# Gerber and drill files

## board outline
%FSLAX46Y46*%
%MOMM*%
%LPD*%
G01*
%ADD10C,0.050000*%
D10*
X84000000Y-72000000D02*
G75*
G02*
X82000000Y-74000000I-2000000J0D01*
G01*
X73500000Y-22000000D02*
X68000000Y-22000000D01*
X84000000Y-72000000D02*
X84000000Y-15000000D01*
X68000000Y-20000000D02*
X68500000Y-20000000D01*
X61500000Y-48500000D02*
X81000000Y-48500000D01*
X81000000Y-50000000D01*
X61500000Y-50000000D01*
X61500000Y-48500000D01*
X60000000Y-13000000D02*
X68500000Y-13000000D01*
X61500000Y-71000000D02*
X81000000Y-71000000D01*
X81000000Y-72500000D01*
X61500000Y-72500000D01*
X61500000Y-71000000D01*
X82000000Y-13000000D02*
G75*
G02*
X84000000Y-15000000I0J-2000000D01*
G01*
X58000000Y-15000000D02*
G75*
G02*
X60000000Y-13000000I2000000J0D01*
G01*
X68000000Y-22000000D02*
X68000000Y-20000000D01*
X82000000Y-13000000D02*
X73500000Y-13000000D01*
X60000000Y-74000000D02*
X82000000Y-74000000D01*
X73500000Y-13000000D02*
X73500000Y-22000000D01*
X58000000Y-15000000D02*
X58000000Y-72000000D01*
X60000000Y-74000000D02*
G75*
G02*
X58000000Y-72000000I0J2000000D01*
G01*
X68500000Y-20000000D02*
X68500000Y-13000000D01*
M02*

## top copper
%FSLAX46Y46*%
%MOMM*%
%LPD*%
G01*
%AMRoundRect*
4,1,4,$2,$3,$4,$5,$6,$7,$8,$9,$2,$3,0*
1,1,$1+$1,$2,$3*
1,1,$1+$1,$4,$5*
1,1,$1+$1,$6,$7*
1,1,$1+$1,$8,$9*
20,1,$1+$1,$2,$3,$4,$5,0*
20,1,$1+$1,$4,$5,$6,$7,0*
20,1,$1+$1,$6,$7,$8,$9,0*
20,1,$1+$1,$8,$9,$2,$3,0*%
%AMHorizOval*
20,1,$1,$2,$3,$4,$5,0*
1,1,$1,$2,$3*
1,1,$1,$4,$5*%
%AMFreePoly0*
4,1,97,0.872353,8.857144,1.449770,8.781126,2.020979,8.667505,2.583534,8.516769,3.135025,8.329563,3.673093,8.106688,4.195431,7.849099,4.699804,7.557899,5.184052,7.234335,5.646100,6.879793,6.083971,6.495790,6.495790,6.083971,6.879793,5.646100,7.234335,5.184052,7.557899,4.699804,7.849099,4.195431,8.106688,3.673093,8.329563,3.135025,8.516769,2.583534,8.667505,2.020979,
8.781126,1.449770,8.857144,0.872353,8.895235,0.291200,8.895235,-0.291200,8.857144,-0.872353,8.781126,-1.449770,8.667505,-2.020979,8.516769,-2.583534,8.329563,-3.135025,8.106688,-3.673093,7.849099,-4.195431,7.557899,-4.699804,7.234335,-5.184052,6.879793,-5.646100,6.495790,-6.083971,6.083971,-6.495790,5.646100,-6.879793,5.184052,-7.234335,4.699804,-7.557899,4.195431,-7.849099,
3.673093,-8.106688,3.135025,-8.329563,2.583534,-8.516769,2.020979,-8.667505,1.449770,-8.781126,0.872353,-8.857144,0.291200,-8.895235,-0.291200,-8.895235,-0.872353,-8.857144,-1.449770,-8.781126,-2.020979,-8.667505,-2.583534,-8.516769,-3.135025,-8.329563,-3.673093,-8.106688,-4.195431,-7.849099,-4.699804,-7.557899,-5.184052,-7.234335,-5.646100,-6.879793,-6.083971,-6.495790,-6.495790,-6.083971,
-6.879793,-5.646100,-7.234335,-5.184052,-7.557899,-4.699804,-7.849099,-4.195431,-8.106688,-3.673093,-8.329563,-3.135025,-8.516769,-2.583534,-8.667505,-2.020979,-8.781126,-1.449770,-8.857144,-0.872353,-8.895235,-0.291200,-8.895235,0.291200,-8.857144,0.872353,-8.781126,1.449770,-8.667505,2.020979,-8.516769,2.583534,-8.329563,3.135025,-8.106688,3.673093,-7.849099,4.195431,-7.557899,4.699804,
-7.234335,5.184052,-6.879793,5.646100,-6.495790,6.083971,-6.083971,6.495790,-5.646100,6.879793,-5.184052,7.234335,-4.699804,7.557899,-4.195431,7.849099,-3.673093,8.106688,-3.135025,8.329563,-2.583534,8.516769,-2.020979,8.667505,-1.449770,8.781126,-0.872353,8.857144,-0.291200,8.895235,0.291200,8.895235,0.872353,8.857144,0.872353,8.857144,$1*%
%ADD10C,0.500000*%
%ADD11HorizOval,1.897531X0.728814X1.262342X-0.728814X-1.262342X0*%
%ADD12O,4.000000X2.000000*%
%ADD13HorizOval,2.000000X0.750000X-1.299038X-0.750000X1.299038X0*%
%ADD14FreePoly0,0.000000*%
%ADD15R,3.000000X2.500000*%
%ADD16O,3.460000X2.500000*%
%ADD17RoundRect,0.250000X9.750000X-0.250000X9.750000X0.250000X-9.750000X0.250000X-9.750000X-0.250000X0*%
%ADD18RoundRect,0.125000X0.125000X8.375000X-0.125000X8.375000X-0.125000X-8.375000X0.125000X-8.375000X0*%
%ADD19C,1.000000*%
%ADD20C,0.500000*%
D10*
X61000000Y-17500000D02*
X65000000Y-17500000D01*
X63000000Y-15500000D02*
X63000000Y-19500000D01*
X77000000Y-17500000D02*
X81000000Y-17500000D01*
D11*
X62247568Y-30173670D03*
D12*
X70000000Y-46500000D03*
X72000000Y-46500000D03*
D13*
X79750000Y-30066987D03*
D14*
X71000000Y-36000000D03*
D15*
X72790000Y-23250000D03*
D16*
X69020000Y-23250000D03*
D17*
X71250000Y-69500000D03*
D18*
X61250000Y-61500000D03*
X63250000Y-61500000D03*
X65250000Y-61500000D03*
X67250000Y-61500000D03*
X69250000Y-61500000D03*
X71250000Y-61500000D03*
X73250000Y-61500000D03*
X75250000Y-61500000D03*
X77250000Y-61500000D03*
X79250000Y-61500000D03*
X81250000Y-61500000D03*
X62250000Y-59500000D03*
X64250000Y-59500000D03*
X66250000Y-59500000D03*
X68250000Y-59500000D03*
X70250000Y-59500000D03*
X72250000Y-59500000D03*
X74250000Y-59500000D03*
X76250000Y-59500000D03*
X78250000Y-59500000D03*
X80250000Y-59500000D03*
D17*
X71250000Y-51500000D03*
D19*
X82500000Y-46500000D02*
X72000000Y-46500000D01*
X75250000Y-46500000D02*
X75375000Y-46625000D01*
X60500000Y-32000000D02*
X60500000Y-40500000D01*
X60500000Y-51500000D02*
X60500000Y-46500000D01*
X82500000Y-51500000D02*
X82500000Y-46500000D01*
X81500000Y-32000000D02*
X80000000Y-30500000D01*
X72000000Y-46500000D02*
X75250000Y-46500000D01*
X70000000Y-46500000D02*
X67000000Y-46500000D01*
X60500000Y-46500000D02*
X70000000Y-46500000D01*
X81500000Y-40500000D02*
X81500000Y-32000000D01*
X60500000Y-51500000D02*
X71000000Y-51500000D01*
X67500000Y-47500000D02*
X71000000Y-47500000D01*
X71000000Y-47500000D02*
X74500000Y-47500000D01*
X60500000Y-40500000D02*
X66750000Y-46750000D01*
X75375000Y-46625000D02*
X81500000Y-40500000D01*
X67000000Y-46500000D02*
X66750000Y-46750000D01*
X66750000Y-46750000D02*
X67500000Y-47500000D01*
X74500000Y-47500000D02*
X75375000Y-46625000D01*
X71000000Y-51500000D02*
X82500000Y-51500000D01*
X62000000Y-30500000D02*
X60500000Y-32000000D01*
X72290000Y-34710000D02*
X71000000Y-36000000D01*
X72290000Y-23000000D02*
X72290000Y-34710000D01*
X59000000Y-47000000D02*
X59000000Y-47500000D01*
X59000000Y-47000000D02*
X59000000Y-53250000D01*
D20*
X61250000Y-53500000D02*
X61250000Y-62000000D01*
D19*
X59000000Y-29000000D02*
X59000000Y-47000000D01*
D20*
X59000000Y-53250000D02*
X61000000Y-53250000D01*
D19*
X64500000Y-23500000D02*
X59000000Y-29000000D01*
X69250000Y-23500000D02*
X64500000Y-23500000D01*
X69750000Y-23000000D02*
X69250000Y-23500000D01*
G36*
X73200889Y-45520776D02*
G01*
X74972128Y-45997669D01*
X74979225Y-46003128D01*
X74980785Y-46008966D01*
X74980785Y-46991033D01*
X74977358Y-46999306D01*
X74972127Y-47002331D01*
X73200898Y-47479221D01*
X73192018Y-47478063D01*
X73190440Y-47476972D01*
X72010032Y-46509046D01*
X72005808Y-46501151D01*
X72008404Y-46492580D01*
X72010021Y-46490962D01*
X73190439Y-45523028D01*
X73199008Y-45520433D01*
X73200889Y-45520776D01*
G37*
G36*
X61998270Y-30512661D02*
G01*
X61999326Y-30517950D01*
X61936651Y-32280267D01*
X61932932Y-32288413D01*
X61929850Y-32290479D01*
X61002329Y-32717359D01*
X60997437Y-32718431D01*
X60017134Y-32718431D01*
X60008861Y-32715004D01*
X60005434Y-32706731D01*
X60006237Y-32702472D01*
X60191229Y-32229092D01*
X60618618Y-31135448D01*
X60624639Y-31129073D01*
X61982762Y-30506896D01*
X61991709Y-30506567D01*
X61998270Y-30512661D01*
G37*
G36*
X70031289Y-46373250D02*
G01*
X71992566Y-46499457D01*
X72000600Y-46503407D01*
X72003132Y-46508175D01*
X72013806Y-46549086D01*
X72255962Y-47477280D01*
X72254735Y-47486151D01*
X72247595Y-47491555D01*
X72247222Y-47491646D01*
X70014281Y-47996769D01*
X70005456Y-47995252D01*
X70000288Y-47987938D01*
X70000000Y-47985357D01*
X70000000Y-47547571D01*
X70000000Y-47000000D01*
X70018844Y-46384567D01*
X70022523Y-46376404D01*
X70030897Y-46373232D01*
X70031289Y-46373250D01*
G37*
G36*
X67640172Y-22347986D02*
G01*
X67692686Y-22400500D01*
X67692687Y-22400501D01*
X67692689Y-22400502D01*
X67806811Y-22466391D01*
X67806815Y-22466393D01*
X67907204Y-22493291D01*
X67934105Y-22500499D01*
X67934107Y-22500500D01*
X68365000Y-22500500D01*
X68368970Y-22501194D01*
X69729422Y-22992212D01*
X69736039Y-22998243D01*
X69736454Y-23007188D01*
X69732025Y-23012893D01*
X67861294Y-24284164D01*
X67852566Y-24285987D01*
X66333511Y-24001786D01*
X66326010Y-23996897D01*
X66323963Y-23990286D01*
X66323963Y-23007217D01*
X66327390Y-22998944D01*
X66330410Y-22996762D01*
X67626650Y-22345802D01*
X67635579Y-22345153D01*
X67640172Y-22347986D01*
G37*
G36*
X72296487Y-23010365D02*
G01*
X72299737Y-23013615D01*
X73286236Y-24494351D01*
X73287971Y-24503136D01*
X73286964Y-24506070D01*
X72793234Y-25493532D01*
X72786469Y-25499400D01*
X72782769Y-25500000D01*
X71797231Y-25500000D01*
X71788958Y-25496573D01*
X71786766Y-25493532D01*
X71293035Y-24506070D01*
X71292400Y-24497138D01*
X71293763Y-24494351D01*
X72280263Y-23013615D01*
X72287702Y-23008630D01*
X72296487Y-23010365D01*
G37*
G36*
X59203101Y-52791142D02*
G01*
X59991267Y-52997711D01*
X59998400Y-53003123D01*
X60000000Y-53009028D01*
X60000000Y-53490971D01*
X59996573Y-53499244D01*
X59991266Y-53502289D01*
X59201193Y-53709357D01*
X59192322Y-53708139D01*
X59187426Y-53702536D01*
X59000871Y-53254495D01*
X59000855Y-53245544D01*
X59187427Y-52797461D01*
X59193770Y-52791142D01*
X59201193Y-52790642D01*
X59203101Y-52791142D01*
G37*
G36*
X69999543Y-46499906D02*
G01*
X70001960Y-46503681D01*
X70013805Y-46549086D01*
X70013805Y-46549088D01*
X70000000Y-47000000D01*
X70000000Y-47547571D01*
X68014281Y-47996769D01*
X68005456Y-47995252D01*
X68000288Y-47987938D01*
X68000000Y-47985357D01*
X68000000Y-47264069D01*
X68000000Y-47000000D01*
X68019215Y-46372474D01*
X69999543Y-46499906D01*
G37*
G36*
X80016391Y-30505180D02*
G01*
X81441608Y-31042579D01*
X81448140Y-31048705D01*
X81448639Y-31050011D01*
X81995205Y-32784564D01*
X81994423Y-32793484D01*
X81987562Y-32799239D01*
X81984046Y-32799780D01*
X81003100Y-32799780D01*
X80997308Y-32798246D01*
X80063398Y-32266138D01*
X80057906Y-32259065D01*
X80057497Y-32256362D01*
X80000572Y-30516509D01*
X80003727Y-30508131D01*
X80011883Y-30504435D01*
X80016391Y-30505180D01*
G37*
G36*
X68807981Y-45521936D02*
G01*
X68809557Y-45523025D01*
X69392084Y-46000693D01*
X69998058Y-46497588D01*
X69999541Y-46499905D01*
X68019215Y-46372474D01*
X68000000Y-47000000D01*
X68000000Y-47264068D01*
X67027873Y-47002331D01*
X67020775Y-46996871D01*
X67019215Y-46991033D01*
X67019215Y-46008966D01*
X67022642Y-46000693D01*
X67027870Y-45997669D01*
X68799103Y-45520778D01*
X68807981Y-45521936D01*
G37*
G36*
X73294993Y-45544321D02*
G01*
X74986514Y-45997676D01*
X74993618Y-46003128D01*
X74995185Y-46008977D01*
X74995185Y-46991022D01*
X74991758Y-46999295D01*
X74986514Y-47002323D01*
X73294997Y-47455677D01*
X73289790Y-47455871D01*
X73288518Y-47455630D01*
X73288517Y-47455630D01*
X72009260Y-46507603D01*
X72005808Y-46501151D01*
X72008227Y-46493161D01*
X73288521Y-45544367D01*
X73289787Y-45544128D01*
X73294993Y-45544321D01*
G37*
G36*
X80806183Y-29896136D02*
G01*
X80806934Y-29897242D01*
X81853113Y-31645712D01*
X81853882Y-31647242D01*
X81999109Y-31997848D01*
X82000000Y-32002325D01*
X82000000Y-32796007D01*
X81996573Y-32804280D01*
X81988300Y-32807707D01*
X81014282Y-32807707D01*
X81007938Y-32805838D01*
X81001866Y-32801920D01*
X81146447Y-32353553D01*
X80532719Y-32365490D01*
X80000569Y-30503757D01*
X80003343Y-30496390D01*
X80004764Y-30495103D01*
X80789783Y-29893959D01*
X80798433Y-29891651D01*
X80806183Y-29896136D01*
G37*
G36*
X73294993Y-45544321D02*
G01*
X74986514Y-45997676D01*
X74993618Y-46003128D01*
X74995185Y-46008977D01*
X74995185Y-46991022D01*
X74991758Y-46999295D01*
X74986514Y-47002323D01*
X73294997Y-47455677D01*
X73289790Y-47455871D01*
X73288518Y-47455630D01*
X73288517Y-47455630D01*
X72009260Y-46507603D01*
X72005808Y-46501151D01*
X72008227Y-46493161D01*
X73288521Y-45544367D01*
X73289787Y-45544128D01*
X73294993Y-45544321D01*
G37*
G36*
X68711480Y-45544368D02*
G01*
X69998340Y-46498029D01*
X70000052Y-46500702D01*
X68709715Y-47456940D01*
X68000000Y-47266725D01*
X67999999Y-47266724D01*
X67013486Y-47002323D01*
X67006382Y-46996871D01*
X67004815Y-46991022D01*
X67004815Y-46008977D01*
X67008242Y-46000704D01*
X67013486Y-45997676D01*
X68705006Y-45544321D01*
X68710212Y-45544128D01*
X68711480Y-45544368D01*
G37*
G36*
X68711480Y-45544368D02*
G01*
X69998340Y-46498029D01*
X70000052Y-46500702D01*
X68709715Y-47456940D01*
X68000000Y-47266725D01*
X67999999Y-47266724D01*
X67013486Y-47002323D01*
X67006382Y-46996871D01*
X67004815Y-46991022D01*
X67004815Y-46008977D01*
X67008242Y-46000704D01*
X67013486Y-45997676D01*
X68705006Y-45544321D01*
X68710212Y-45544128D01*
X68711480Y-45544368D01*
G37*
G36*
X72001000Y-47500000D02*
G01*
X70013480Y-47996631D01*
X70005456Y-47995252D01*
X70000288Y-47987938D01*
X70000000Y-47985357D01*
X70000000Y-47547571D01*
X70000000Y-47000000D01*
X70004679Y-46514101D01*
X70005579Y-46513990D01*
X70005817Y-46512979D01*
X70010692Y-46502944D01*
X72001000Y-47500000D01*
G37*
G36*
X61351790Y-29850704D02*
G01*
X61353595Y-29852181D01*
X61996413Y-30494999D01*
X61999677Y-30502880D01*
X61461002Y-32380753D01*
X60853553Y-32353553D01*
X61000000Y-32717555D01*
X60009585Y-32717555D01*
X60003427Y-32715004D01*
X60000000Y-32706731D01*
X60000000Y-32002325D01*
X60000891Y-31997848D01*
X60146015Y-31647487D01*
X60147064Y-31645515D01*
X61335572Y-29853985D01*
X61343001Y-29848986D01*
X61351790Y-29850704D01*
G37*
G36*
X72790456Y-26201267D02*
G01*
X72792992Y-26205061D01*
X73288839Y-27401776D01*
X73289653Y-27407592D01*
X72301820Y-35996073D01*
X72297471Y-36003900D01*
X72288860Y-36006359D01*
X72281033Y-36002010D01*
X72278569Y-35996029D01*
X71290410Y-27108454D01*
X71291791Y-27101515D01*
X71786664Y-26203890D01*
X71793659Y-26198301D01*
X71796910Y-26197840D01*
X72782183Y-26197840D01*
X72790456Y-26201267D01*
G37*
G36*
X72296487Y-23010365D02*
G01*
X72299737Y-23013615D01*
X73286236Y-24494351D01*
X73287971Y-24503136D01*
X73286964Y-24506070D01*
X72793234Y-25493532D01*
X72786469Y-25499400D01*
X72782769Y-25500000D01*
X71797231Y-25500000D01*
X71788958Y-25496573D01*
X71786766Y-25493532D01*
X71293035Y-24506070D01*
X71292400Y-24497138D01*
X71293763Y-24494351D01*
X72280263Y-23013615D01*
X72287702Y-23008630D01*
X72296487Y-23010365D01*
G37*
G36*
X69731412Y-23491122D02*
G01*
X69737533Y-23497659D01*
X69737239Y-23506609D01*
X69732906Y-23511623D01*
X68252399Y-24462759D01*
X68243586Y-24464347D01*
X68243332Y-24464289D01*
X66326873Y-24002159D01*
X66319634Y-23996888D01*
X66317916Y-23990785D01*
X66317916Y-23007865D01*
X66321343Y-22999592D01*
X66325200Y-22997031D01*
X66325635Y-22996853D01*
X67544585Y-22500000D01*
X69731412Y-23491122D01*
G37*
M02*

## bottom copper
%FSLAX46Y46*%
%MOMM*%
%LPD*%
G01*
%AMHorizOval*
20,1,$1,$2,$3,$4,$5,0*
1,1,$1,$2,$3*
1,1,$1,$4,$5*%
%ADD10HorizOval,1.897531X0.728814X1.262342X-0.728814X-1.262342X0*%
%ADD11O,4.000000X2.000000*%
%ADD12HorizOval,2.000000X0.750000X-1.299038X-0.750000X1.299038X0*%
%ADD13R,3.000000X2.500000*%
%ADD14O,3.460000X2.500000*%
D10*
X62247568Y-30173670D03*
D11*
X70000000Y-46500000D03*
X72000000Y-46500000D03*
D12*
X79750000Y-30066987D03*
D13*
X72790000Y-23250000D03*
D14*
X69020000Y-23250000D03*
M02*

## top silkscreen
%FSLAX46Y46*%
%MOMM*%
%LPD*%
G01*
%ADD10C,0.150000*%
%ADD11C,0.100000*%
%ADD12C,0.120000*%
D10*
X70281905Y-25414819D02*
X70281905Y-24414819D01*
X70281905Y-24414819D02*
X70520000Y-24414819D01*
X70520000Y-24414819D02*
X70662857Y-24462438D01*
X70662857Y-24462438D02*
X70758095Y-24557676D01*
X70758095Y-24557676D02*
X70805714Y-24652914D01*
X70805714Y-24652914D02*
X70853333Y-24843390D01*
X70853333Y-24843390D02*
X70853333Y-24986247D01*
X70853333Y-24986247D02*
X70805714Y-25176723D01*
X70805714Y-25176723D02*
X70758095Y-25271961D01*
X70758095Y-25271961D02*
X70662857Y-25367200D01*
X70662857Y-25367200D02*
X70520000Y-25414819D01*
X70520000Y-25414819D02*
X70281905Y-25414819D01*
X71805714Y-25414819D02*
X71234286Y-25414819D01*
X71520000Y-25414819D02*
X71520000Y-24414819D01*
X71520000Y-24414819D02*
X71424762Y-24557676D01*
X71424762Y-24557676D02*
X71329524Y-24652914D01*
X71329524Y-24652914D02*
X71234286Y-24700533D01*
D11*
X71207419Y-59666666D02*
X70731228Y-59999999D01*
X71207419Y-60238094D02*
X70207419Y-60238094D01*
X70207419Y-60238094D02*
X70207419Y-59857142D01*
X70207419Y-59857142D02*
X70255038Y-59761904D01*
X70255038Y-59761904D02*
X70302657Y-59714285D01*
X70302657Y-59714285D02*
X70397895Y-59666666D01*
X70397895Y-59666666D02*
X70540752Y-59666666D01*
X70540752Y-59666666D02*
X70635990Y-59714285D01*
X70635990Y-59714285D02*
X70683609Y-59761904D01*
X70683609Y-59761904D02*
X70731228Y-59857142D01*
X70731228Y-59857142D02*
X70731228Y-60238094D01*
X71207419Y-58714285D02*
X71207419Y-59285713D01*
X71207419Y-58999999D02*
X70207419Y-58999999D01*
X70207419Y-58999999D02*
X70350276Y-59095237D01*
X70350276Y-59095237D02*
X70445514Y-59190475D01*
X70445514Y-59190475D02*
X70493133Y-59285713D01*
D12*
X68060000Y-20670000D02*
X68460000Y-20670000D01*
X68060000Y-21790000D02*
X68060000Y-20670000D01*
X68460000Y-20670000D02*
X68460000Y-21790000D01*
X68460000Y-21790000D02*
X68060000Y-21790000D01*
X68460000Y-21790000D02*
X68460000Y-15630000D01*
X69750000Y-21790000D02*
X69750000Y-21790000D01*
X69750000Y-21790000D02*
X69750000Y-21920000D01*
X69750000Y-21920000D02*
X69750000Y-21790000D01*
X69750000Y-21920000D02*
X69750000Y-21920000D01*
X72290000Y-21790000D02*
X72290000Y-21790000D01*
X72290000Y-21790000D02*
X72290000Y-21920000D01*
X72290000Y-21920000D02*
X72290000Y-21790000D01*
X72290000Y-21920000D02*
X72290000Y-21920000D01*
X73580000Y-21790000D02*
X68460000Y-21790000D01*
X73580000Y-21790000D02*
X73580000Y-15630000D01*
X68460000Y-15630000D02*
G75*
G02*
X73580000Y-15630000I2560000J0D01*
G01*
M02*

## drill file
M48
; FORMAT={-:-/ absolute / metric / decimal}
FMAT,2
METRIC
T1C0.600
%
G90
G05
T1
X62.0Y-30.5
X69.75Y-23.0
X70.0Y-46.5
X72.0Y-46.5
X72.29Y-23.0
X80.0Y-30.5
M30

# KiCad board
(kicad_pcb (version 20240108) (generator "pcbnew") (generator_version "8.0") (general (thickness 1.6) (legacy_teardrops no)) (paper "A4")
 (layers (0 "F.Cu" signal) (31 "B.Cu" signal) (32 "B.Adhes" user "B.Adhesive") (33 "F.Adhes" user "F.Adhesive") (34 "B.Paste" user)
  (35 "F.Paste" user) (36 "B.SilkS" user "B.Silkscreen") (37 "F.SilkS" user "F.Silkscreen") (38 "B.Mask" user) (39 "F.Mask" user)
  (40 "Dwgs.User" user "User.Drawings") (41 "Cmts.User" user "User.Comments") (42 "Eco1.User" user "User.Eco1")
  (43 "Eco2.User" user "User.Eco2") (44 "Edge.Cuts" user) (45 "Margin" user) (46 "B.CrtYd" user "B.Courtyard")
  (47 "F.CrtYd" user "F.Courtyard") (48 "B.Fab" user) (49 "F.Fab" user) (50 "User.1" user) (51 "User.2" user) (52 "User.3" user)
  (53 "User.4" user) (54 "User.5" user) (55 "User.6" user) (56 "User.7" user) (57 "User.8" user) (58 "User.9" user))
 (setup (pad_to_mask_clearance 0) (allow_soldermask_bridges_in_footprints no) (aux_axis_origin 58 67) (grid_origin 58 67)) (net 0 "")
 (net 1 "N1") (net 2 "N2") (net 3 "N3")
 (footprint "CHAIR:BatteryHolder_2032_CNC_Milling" (layer "F.Cu") (at 71 36)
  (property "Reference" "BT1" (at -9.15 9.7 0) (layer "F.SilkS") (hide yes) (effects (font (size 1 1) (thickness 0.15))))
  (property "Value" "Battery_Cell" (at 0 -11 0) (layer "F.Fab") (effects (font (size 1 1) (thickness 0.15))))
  (pad "1" thru_hole oval (at -9 -5.5 60) (size 4.812786 1.897531) (drill 0.6 (offset 0.406394 0.051235)) (layers "*.Cu" "*.Mask")
   (remove_unused_layers no) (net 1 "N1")
   (teardrops (best_length_ratio 0.5) (max_length 1) (best_width_ratio 1) (max_width 2) (curve_points 0) (filter_ratio 0.9) (enabled yes)
    (allow_two_segments yes) (prefer_zone_connections yes)))
  (pad "1" thru_hole oval (at -1 10.5) (size 4 2) (drill 0.6) (layers "*.Cu" "*.Mask") (remove_unused_layers no) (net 1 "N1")
   (teardrops (best_length_ratio 0.5) (max_length 1) (best_width_ratio 1) (max_width 2) (curve_points 0) (filter_ratio 0.9) (enabled yes)
    (allow_two_segments yes) (prefer_zone_connections yes)))
  (pad "1" thru_hole oval (at 1 10.5) (size 4 2) (drill 0.6) (layers "*.Cu" "*.Mask") (remove_unused_layers no) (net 1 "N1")
   (teardrops (best_length_ratio 0.5) (max_length 1) (best_width_ratio 1) (max_width 2) (curve_points 0) (filter_ratio 0.9) (enabled yes)
    (allow_two_segments yes) (prefer_zone_connections yes)))
  (pad "1" thru_hole oval (at 9 -5.5 300) (size 5 2) (drill 0.6 (offset -0.5 0)) (layers "*.Cu" "*.Mask") (remove_unused_layers no)
   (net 1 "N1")
   (teardrops (best_length_ratio 0.5) (max_length 1) (best_width_ratio 1) (max_width 2) (curve_points 0) (filter_ratio 0.9) (enabled yes)
    (allow_two_segments yes) (prefer_zone_connections yes)))
  (pad "2" smd custom (at 0 0) (size 17.8 17.8) (layers "F.Cu" "F.Mask") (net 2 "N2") (thermal_bridge_angle 90)
   (options (clearance outline) (anchor circle)) (primitives)
   (teardrops (best_length_ratio 0.5) (max_length 1) (best_width_ratio 1) (max_width 2) (curve_points 0) (filter_ratio 0.9) (enabled yes)
    (allow_two_segments yes) (prefer_zone_connections yes))))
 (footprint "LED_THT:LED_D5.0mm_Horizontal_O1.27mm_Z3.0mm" (layer "F.Cu") (at 72.29 23 180)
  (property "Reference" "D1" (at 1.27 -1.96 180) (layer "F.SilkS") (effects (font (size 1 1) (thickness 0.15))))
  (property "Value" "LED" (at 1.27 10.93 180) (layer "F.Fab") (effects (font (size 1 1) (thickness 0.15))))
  (fp_line (start 4.23 2.33) (end 3.83 2.33) (stroke (width 0.12) (type solid)) (layer "F.SilkS"))
  (fp_line (start 4.23 1.21) (end 4.23 2.33) (stroke (width 0.12) (type solid)) (layer "F.SilkS"))
  (fp_line (start 3.83 2.33) (end 3.83 1.21) (stroke (width 0.12) (type solid)) (layer "F.SilkS"))
  (fp_line (start 3.83 1.21) (end 4.23 1.21) (stroke (width 0.12) (type solid)) (layer "F.SilkS"))
  (fp_line (start 3.83 1.21) (end 3.83 7.37) (stroke (width 0.12) (type solid)) (layer "F.SilkS"))
  (fp_line (start 2.54 1.21) (end 2.54 1.21) (stroke (width 0.12) (type solid)) (layer "F.SilkS"))
  (fp_line (start 2.54 1.21) (end 2.54 1.08) (stroke (width 0.12) (type solid)) (layer "F.SilkS"))
  (fp_line (start 2.54 1.08) (end 2.54 1.21) (stroke (width 0.12) (type solid)) (layer "F.SilkS"))
  (fp_line (start 2.54 1.08) (end 2.54 1.08) (stroke (width 0.12) (type solid)) (layer "F.SilkS"))
  (fp_line (start 0 1.21) (end 0 1.21) (stroke (width 0.12) (type solid)) (layer "F.SilkS"))
  (fp_line (start 0 1.21) (end 0 1.08) (stroke (width 0.12) (type solid)) (layer "F.SilkS"))
  (fp_line (start 0 1.08) (end 0 1.21) (stroke (width 0.12) (type solid)) (layer "F.SilkS"))
  (fp_line (start 0 1.08) (end 0 1.08) (stroke (width 0.12) (type solid)) (layer "F.SilkS"))
  (fp_line (start -1.29 1.21) (end 3.83 1.21) (stroke (width 0.12) (type solid)) (layer "F.SilkS"))
  (fp_line (start -1.29 1.21) (end -1.29 7.37) (stroke (width 0.12) (type solid)) (layer "F.SilkS"))
  (fp_arc (start 3.83 7.37) (mid 1.27 9.93) (end -1.29 7.37) (stroke (width 0.12) (type solid)) (layer "F.SilkS"))
  (pad "1" thru_hole rect (at 0 0 180) (size 3 2.5) (drill 0.6 (offset -0.5 -0.25)) (layers "*.Cu" "*.Mask") (remove_unused_layers no)
   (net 2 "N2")
   (teardrops (best_length_ratio 0.5) (max_length 1) (best_width_ratio 1) (max_width 2) (curve_points 0) (filter_ratio 0.9) (enabled yes)
    (allow_two_segments yes) (prefer_zone_connections yes)))
  (pad "2" thru_hole oval (at 2.54 0 180) (size 3.46 2.5) (drill 0.6 (offset 0.73 -0.25)) (layers "*.Cu" "*.Mask") (remove_unused_layers no)
   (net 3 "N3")
   (teardrops (best_length_ratio 0.5) (max_length 1) (best_width_ratio 1) (max_width 2) (curve_points 0) (filter_ratio 0.9) (enabled yes)
    (allow_two_segments yes) (prefer_zone_connections yes))))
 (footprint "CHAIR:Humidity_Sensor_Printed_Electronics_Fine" (layer "F.Cu") (at 71.25 59.5 90)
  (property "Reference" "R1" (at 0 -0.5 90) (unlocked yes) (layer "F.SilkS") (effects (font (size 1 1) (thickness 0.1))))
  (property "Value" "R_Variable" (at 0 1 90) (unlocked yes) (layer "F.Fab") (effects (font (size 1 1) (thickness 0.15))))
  (pad "1" smd roundrect (at -10 0 90) (size 1 20) (layers "F.Cu" "F.Mask") (roundrect_rratio 0.25) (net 3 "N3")
   (teardrops (best_length_ratio 0.5) (max_length 1) (best_width_ratio 1) (max_width 2) (curve_points 0) (filter_ratio 0.9) (enabled yes)
    (allow_two_segments yes) (prefer_zone_connections yes)))
  (pad "1" smd roundrect (at -2 -10 180) (size 0.5 17) (layers "F.Cu" "F.Mask") (roundrect_rratio 0.25) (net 3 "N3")
   (teardrops (best_length_ratio 0.5) (max_length 1) (best_width_ratio 1) (max_width 2) (curve_points 0) (filter_ratio 0.9) (enabled yes)
    (allow_two_segments yes) (prefer_zone_connections yes)))
  (pad "1" smd roundrect (at -2 -8 180) (size 0.5 17) (layers "F.Cu" "F.Mask") (roundrect_rratio 0.25) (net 3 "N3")
   (teardrops (best_length_ratio 0.5) (max_length 1) (best_width_ratio 1) (max_width 2) (curve_points 0) (filter_ratio 0.9) (enabled yes)
    (allow_two_segments yes) (prefer_zone_connections yes)))
  (pad "1" smd roundrect (at -2 -6 180) (size 0.5 17) (layers "F.Cu" "F.Mask") (roundrect_rratio 0.25) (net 3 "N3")
   (teardrops (best_length_ratio 0.5) (max_length 1) (best_width_ratio 1) (max_width 2) (curve_points 0) (filter_ratio 0.9) (enabled yes)
    (allow_two_segments yes) (prefer_zone_connections yes)))
  (pad "1" smd roundrect (at -2 -4 180) (size 0.5 17) (layers "F.Cu" "F.Mask") (roundrect_rratio 0.25) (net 3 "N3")
   (teardrops (best_length_ratio 0.5) (max_length 1) (best_width_ratio 1) (max_width 2) (curve_points 0) (filter_ratio 0.9) (enabled yes)
    (allow_two_segments yes) (prefer_zone_connections yes)))
  (pad "1" smd roundrect (at -2 -2 180) (size 0.5 17) (layers "F.Cu" "F.Mask") (roundrect_rratio 0.25) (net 3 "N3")
   (teardrops (best_length_ratio 0.5) (max_length 1) (best_width_ratio 1) (max_width 2) (curve_points 0) (filter_ratio 0.9) (enabled yes)
    (allow_two_segments yes) (prefer_zone_connections yes)))
  (pad "1" smd roundrect (at -2 0 180) (size 0.5 17) (layers "F.Cu" "F.Mask") (roundrect_rratio 0.25) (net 3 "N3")
   (teardrops (best_length_ratio 0.5) (max_length 1) (best_width_ratio 1) (max_width 2) (curve_points 0) (filter_ratio 0.9) (enabled yes)
    (allow_two_segments yes) (prefer_zone_connections yes)))
  (pad "1" smd roundrect (at -2 2 180) (size 0.5 17) (layers "F.Cu" "F.Mask") (roundrect_rratio 0.25) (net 3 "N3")
   (teardrops (best_length_ratio 0.5) (max_length 1) (best_width_ratio 1) (max_width 2) (curve_points 0) (filter_ratio 0.9) (enabled yes)
    (allow_two_segments yes) (prefer_zone_connections yes)))
  (pad "1" smd roundrect (at -2 4 180) (size 0.5 17) (layers "F.Cu" "F.Mask") (roundrect_rratio 0.25) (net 3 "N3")
   (teardrops (best_length_ratio 0.5) (max_length 1) (best_width_ratio 1) (max_width 2) (curve_points 0) (filter_ratio 0.9) (enabled yes)
    (allow_two_segments yes) (prefer_zone_connections yes)))
  (pad "1" smd roundrect (at -2 6 180) (size 0.5 17) (layers "F.Cu" "F.Mask") (roundrect_rratio 0.25) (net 3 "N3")
   (teardrops (best_length_ratio 0.5) (max_length 1) (best_width_ratio 1) (max_width 2) (curve_points 0) (filter_ratio 0.9) (enabled yes)
    (allow_two_segments yes) (prefer_zone_connections yes)))
  (pad "1" smd roundrect (at -2 8 180) (size 0.5 17) (layers "F.Cu" "F.Mask") (roundrect_rratio 0.25) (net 3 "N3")
   (teardrops (best_length_ratio 0.5) (max_length 1) (best_width_ratio 1) (max_width 2) (curve_points 0) (filter_ratio 0.9) (enabled yes)
    (allow_two_segments yes) (prefer_zone_connections yes)))
  (pad "1" smd roundrect (at -2 10 180) (size 0.5 17) (layers "F.Cu" "F.Mask") (roundrect_rratio 0.25) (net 3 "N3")
   (teardrops (best_length_ratio 0.5) (max_length 1) (best_width_ratio 1) (max_width 2) (curve_points 0) (filter_ratio 0.9) (enabled yes)
    (allow_two_segments yes) (prefer_zone_connections yes)))
  (pad "2" smd roundrect (at 0 -9 180) (size 0.5 17) (layers "F.Cu" "F.Mask") (roundrect_rratio 0.25) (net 1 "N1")
   (teardrops (best_length_ratio 0.5) (max_length 1) (best_width_ratio 1) (max_width 2) (curve_points 0) (filter_ratio 0.9) (enabled yes)
    (allow_two_segments yes) (prefer_zone_connections yes)))
  (pad "2" smd roundrect (at 0 -7 180) (size 0.5 17) (layers "F.Cu" "F.Mask") (roundrect_rratio 0.25) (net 1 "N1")
   (teardrops (best_length_ratio 0.5) (max_length 1) (best_width_ratio 1) (max_width 2) (curve_points 0) (filter_ratio 0.9) (enabled yes)
    (allow_two_segments yes) (prefer_zone_connections yes)))
  (pad "2" smd roundrect (at 0 -5 180) (size 0.5 17) (layers "F.Cu" "F.Mask") (roundrect_rratio 0.25) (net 1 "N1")
   (teardrops (best_length_ratio 0.5) (max_length 1) (best_width_ratio 1) (max_width 2) (curve_points 0) (filter_ratio 0.9) (enabled yes)
    (allow_two_segments yes) (prefer_zone_connections yes)))
  (pad "2" smd roundrect (at 0 -3 180) (size 0.5 17) (layers "F.Cu" "F.Mask") (roundrect_rratio 0.25) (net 1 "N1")
   (teardrops (best_length_ratio 0.5) (max_length 1) (best_width_ratio 1) (max_width 2) (curve_points 0) (filter_ratio 0.9) (enabled yes)
    (allow_two_segments yes) (prefer_zone_connections yes)))
  (pad "2" smd roundrect (at 0 -1 180) (size 0.5 17) (layers "F.Cu" "F.Mask") (roundrect_rratio 0.25) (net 1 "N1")
   (teardrops (best_length_ratio 0.5) (max_length 1) (best_width_ratio 1) (max_width 2) (curve_points 0) (filter_ratio 0.9) (enabled yes)
    (allow_two_segments yes) (prefer_zone_connections yes)))
  (pad "2" smd roundrect (at 0 1 180) (size 0.5 17) (layers "F.Cu" "F.Mask") (roundrect_rratio 0.25) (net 1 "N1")
   (teardrops (best_length_ratio 0.5) (max_length 1) (best_width_ratio 1) (max_width 2) (curve_points 0) (filter_ratio 0.9) (enabled yes)
    (allow_two_segments yes) (prefer_zone_connections yes)))
  (pad "2" smd roundrect (at 0 3 180) (size 0.5 17) (layers "F.Cu" "F.Mask") (roundrect_rratio 0.25) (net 1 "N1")
   (teardrops (best_length_ratio 0.5) (max_length 1) (best_width_ratio 1) (max_width 2) (curve_points 0) (filter_ratio 0.9) (enabled yes)
    (allow_two_segments yes) (prefer_zone_connections yes)))
  (pad "2" smd roundrect (at 0 5 180) (size 0.5 17) (layers "F.Cu" "F.Mask") (roundrect_rratio 0.25) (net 1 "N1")
   (teardrops (best_length_ratio 0.5) (max_length 1) (best_width_ratio 1) (max_width 2) (curve_points 0) (filter_ratio 0.9) (enabled yes)
    (allow_two_segments yes) (prefer_zone_connections yes)))
  (pad "2" smd roundrect (at 0 7 180) (size 0.5 17) (layers "F.Cu" "F.Mask") (roundrect_rratio 0.25) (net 1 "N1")
   (teardrops (best_length_ratio 0.5) (max_length 1) (best_width_ratio 1) (max_width 2) (curve_points 0) (filter_ratio 0.9) (enabled yes)
    (allow_two_segments yes) (prefer_zone_connections yes)))
  (pad "2" smd roundrect (at 0 9 180) (size 0.5 17) (layers "F.Cu" "F.Mask") (roundrect_rratio 0.25) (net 1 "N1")
   (teardrops (best_length_ratio 0.5) (max_length 1) (best_width_ratio 1) (max_width 2) (curve_points 0) (filter_ratio 0.9) (enabled yes)
    (allow_two_segments yes) (prefer_zone_connections yes)))
  (pad "2" smd roundrect (at 8 0 90) (size 1 20) (layers "F.Cu" "F.Mask") (roundrect_rratio 0.25) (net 1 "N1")
   (teardrops (best_length_ratio 0.5) (max_length 1) (best_width_ratio 1) (max_width 2) (curve_points 0) (filter_ratio 0.9) (enabled yes)
    (allow_two_segments yes) (prefer_zone_connections yes))))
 (gr_line (start 61 17.5) (end 65 17.5) (stroke (width 0.5) (type default)) (layer "F.Cu"))
 (gr_line (start 63 15.5) (end 63 19.5) (stroke (width 0.5) (type default)) (layer "F.Cu"))
 (gr_line (start 77 17.5) (end 81 17.5) (stroke (width 0.5) (type default)) (layer "F.Cu"))
 (gr_arc (start 84 72) (mid 83.414214 73.414214) (end 82 74) (stroke (width 0.05) (type default)) (layer "Edge.Cuts"))
 (gr_line (start 73.5 22) (end 68 22) (stroke (width 0.05) (type default)) (layer "Edge.Cuts"))
 (gr_line (start 84 72) (end 84 15) (stroke (width 0.05) (type default)) (layer "Edge.Cuts"))
 (gr_line (start 68 20) (end 68.5 20) (stroke (width 0.05) (type default)) (layer "Edge.Cuts"))
 (gr_rect (start 61.5 48.5) (end 81 50) (stroke (width 0.05) (type default)) (fill none) (layer "Edge.Cuts"))
 (gr_line (start 60 13) (end 68.5 13) (stroke (width 0.05) (type default)) (layer "Edge.Cuts"))
 (gr_rect (start 61.5 71) (end 81 72.5) (stroke (width 0.05) (type default)) (fill none) (layer "Edge.Cuts"))
 (gr_arc (start 82 13) (mid 83.414214 13.585786) (end 84 15) (stroke (width 0.05) (type default)) (layer "Edge.Cuts"))
 (gr_arc (start 58 15) (mid 58.585786 13.585786) (end 60 13) (stroke (width 0.05) (type default)) (layer "Edge.Cuts"))
 (gr_line (start 68 22) (end 68 20) (stroke (width 0.05) (type default)) (layer "Edge.Cuts"))
 (gr_line (start 82 13) (end 73.5 13) (stroke (width 0.05) (type default)) (layer "Edge.Cuts"))
 (gr_line (start 60 74) (end 82 74) (stroke (width 0.05) (type default)) (layer "Edge.Cuts"))
 (gr_line (start 73.5 13) (end 73.5 22) (stroke (width 0.05) (type default)) (layer "Edge.Cuts"))
 (gr_line (start 58 15) (end 58 72) (stroke (width 0.05) (type default)) (layer "Edge.Cuts"))
 (gr_arc (start 60 74) (mid 58.585786 73.414214) (end 58 72) (stroke (width 0.05) (type default)) (layer "Edge.Cuts"))
 (gr_line (start 68.5 20) (end 68.5 13) (stroke (width 0.05) (type default)) (layer "Edge.Cuts"))
 (segment (start 82.5 46.5) (end 72 46.5) (width 1) (layer "F.Cu") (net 1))
 (segment (start 75.25 46.5) (end 75.375 46.625) (width 1) (layer "F.Cu") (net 1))
 (segment (start 60.5 32) (end 60.5 40.5) (width 1) (layer "F.Cu") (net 1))
 (segment (start 60.5 51.5) (end 60.5 46.5) (width 1) (layer "F.Cu") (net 1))
 (segment (start 82.5 51.5) (end 82.5 46.5) (width 1) (layer "F.Cu") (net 1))
 (segment (start 81.5 32) (end 80 30.5) (width 1) (layer "F.Cu") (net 1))
 (segment (start 72 46.5) (end 75.25 46.5) (width 1) (layer "F.Cu") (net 1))
 (segment (start 70 46.5) (end 67 46.5) (width 1) (layer "F.Cu") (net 1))
 (segment (start 60.5 46.5) (end 70 46.5) (width 1) (layer "F.Cu") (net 1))
 (segment (start 81.5 40.5) (end 81.5 32) (width 1) (layer "F.Cu") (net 1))
 (segment (start 60.5 51.5) (end 71 51.5) (width 1) (layer "F.Cu") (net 1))
 (segment (start 67.5 47.5) (end 71 47.5) (width 1) (layer "F.Cu") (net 1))
 (segment (start 71 47.5) (end 74.5 47.5) (width 1) (layer "F.Cu") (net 1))
 (segment (start 60.5 40.5) (end 66.75 46.75) (width 1) (layer "F.Cu") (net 1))
 (segment (start 75.375 46.625) (end 81.5 40.5) (width 1) (layer "F.Cu") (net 1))
 (segment (start 67 46.5) (end 66.75 46.75) (width 1) (layer "F.Cu") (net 1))
 (segment (start 66.75 46.75) (end 67.5 47.5) (width 1) (layer "F.Cu") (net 1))
 (segment (start 74.5 47.5) (end 75.375 46.625) (width 1) (layer "F.Cu") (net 1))
 (segment (start 71 51.5) (end 82.5 51.5) (width 1) (layer "F.Cu") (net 1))
 (segment (start 62 30.5) (end 60.5 32) (width 1) (layer "F.Cu") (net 1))
 (segment (start 72.29 34.71) (end 71 36) (width 1) (layer "F.Cu") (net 2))
 (segment (start 72.29 23) (end 72.29 34.71) (width 1) (layer "F.Cu") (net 2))
 (segment (start 59 47) (end 59 47.5) (width 1) (layer "F.Cu") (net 3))
 (segment (start 59 47) (end 59 53.25) (width 1) (layer "F.Cu") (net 3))
 (segment (start 61.25 53.5) (end 61.25 62) (width 0.5) (layer "F.Cu") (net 3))
 (segment (start 59 29) (end 59 47) (width 1) (layer "F.Cu") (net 3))
 (segment (start 59 53.25) (end 61 53.25) (width 0.5) (layer "F.Cu") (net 3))
 (segment (start 64.5 23.5) (end 59 29) (width 1) (layer "F.Cu") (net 3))
 (segment (start 69.25 23.5) (end 64.5 23.5) (width 1) (layer "F.Cu") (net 3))
 (segment (start 69.75 23) (end 69.25 23.5) (width 1) (layer "F.Cu") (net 3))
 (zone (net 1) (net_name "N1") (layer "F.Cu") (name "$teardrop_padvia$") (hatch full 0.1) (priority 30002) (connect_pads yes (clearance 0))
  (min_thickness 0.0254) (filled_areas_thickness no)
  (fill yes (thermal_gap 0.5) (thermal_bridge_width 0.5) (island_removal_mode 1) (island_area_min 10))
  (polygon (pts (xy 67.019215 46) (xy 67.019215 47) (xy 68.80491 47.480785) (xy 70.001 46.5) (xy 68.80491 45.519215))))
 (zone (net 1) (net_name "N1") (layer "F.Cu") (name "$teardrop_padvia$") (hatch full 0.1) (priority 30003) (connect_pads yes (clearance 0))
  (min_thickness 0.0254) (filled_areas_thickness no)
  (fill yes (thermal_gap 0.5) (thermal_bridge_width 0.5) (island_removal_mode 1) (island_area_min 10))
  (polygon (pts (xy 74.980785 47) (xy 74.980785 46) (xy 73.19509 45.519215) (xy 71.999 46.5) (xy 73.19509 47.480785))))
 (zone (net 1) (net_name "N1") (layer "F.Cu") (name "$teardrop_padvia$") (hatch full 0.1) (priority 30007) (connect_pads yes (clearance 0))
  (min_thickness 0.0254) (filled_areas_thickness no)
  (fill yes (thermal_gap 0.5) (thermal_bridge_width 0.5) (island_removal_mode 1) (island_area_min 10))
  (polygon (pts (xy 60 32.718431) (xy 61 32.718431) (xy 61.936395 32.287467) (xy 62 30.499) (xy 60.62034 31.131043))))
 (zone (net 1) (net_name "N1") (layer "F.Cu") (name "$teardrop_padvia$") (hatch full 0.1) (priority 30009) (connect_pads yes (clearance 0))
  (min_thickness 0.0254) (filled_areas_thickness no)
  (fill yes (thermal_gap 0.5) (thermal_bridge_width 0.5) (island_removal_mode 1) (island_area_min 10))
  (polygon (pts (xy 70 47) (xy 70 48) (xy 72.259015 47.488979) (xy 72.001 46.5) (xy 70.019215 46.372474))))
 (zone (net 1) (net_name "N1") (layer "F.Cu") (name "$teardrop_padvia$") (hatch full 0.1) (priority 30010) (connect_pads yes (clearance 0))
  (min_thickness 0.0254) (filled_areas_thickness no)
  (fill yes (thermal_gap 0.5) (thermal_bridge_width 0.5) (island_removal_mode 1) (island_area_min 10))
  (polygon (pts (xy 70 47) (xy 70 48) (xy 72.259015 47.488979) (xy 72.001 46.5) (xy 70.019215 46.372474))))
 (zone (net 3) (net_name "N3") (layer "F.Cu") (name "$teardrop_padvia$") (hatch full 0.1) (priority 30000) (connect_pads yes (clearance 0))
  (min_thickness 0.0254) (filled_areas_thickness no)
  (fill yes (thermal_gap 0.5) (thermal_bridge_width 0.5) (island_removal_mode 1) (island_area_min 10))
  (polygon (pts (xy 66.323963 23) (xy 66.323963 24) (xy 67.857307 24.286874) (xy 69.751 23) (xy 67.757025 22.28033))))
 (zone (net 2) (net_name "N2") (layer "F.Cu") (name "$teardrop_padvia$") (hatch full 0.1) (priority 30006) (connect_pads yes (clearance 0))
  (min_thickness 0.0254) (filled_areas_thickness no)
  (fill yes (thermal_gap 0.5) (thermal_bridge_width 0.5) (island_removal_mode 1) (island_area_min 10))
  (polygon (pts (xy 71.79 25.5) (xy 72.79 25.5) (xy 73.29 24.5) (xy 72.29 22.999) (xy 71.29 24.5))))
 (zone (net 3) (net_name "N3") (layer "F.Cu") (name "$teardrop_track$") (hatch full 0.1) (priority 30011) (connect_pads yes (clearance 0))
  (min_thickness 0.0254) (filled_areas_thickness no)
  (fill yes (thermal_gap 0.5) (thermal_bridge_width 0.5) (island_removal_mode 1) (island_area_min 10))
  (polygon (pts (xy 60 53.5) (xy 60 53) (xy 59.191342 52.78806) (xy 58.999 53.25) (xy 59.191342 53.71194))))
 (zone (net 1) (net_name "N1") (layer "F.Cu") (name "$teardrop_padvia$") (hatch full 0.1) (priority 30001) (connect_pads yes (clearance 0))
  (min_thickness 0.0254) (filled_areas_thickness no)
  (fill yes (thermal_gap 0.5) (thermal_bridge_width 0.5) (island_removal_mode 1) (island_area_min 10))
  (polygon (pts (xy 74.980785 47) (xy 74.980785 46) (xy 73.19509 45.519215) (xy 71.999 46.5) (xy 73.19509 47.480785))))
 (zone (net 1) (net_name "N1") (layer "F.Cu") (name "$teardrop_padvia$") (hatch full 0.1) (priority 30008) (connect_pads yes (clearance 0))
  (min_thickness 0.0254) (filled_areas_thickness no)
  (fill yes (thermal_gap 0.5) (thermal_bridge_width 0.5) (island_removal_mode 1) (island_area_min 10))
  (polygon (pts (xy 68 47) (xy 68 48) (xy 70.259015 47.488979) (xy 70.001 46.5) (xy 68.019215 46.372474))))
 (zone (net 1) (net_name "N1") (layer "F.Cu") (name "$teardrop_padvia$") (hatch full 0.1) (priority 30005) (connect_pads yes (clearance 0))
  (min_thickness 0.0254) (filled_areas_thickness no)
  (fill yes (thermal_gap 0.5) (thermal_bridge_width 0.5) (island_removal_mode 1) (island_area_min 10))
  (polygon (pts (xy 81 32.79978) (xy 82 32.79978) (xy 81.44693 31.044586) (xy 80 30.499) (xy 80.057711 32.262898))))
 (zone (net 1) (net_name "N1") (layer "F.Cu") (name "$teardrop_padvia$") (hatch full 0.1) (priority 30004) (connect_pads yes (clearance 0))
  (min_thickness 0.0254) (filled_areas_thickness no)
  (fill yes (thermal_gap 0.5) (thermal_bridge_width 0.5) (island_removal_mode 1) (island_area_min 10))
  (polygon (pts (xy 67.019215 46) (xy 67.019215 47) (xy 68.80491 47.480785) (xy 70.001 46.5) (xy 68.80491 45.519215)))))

